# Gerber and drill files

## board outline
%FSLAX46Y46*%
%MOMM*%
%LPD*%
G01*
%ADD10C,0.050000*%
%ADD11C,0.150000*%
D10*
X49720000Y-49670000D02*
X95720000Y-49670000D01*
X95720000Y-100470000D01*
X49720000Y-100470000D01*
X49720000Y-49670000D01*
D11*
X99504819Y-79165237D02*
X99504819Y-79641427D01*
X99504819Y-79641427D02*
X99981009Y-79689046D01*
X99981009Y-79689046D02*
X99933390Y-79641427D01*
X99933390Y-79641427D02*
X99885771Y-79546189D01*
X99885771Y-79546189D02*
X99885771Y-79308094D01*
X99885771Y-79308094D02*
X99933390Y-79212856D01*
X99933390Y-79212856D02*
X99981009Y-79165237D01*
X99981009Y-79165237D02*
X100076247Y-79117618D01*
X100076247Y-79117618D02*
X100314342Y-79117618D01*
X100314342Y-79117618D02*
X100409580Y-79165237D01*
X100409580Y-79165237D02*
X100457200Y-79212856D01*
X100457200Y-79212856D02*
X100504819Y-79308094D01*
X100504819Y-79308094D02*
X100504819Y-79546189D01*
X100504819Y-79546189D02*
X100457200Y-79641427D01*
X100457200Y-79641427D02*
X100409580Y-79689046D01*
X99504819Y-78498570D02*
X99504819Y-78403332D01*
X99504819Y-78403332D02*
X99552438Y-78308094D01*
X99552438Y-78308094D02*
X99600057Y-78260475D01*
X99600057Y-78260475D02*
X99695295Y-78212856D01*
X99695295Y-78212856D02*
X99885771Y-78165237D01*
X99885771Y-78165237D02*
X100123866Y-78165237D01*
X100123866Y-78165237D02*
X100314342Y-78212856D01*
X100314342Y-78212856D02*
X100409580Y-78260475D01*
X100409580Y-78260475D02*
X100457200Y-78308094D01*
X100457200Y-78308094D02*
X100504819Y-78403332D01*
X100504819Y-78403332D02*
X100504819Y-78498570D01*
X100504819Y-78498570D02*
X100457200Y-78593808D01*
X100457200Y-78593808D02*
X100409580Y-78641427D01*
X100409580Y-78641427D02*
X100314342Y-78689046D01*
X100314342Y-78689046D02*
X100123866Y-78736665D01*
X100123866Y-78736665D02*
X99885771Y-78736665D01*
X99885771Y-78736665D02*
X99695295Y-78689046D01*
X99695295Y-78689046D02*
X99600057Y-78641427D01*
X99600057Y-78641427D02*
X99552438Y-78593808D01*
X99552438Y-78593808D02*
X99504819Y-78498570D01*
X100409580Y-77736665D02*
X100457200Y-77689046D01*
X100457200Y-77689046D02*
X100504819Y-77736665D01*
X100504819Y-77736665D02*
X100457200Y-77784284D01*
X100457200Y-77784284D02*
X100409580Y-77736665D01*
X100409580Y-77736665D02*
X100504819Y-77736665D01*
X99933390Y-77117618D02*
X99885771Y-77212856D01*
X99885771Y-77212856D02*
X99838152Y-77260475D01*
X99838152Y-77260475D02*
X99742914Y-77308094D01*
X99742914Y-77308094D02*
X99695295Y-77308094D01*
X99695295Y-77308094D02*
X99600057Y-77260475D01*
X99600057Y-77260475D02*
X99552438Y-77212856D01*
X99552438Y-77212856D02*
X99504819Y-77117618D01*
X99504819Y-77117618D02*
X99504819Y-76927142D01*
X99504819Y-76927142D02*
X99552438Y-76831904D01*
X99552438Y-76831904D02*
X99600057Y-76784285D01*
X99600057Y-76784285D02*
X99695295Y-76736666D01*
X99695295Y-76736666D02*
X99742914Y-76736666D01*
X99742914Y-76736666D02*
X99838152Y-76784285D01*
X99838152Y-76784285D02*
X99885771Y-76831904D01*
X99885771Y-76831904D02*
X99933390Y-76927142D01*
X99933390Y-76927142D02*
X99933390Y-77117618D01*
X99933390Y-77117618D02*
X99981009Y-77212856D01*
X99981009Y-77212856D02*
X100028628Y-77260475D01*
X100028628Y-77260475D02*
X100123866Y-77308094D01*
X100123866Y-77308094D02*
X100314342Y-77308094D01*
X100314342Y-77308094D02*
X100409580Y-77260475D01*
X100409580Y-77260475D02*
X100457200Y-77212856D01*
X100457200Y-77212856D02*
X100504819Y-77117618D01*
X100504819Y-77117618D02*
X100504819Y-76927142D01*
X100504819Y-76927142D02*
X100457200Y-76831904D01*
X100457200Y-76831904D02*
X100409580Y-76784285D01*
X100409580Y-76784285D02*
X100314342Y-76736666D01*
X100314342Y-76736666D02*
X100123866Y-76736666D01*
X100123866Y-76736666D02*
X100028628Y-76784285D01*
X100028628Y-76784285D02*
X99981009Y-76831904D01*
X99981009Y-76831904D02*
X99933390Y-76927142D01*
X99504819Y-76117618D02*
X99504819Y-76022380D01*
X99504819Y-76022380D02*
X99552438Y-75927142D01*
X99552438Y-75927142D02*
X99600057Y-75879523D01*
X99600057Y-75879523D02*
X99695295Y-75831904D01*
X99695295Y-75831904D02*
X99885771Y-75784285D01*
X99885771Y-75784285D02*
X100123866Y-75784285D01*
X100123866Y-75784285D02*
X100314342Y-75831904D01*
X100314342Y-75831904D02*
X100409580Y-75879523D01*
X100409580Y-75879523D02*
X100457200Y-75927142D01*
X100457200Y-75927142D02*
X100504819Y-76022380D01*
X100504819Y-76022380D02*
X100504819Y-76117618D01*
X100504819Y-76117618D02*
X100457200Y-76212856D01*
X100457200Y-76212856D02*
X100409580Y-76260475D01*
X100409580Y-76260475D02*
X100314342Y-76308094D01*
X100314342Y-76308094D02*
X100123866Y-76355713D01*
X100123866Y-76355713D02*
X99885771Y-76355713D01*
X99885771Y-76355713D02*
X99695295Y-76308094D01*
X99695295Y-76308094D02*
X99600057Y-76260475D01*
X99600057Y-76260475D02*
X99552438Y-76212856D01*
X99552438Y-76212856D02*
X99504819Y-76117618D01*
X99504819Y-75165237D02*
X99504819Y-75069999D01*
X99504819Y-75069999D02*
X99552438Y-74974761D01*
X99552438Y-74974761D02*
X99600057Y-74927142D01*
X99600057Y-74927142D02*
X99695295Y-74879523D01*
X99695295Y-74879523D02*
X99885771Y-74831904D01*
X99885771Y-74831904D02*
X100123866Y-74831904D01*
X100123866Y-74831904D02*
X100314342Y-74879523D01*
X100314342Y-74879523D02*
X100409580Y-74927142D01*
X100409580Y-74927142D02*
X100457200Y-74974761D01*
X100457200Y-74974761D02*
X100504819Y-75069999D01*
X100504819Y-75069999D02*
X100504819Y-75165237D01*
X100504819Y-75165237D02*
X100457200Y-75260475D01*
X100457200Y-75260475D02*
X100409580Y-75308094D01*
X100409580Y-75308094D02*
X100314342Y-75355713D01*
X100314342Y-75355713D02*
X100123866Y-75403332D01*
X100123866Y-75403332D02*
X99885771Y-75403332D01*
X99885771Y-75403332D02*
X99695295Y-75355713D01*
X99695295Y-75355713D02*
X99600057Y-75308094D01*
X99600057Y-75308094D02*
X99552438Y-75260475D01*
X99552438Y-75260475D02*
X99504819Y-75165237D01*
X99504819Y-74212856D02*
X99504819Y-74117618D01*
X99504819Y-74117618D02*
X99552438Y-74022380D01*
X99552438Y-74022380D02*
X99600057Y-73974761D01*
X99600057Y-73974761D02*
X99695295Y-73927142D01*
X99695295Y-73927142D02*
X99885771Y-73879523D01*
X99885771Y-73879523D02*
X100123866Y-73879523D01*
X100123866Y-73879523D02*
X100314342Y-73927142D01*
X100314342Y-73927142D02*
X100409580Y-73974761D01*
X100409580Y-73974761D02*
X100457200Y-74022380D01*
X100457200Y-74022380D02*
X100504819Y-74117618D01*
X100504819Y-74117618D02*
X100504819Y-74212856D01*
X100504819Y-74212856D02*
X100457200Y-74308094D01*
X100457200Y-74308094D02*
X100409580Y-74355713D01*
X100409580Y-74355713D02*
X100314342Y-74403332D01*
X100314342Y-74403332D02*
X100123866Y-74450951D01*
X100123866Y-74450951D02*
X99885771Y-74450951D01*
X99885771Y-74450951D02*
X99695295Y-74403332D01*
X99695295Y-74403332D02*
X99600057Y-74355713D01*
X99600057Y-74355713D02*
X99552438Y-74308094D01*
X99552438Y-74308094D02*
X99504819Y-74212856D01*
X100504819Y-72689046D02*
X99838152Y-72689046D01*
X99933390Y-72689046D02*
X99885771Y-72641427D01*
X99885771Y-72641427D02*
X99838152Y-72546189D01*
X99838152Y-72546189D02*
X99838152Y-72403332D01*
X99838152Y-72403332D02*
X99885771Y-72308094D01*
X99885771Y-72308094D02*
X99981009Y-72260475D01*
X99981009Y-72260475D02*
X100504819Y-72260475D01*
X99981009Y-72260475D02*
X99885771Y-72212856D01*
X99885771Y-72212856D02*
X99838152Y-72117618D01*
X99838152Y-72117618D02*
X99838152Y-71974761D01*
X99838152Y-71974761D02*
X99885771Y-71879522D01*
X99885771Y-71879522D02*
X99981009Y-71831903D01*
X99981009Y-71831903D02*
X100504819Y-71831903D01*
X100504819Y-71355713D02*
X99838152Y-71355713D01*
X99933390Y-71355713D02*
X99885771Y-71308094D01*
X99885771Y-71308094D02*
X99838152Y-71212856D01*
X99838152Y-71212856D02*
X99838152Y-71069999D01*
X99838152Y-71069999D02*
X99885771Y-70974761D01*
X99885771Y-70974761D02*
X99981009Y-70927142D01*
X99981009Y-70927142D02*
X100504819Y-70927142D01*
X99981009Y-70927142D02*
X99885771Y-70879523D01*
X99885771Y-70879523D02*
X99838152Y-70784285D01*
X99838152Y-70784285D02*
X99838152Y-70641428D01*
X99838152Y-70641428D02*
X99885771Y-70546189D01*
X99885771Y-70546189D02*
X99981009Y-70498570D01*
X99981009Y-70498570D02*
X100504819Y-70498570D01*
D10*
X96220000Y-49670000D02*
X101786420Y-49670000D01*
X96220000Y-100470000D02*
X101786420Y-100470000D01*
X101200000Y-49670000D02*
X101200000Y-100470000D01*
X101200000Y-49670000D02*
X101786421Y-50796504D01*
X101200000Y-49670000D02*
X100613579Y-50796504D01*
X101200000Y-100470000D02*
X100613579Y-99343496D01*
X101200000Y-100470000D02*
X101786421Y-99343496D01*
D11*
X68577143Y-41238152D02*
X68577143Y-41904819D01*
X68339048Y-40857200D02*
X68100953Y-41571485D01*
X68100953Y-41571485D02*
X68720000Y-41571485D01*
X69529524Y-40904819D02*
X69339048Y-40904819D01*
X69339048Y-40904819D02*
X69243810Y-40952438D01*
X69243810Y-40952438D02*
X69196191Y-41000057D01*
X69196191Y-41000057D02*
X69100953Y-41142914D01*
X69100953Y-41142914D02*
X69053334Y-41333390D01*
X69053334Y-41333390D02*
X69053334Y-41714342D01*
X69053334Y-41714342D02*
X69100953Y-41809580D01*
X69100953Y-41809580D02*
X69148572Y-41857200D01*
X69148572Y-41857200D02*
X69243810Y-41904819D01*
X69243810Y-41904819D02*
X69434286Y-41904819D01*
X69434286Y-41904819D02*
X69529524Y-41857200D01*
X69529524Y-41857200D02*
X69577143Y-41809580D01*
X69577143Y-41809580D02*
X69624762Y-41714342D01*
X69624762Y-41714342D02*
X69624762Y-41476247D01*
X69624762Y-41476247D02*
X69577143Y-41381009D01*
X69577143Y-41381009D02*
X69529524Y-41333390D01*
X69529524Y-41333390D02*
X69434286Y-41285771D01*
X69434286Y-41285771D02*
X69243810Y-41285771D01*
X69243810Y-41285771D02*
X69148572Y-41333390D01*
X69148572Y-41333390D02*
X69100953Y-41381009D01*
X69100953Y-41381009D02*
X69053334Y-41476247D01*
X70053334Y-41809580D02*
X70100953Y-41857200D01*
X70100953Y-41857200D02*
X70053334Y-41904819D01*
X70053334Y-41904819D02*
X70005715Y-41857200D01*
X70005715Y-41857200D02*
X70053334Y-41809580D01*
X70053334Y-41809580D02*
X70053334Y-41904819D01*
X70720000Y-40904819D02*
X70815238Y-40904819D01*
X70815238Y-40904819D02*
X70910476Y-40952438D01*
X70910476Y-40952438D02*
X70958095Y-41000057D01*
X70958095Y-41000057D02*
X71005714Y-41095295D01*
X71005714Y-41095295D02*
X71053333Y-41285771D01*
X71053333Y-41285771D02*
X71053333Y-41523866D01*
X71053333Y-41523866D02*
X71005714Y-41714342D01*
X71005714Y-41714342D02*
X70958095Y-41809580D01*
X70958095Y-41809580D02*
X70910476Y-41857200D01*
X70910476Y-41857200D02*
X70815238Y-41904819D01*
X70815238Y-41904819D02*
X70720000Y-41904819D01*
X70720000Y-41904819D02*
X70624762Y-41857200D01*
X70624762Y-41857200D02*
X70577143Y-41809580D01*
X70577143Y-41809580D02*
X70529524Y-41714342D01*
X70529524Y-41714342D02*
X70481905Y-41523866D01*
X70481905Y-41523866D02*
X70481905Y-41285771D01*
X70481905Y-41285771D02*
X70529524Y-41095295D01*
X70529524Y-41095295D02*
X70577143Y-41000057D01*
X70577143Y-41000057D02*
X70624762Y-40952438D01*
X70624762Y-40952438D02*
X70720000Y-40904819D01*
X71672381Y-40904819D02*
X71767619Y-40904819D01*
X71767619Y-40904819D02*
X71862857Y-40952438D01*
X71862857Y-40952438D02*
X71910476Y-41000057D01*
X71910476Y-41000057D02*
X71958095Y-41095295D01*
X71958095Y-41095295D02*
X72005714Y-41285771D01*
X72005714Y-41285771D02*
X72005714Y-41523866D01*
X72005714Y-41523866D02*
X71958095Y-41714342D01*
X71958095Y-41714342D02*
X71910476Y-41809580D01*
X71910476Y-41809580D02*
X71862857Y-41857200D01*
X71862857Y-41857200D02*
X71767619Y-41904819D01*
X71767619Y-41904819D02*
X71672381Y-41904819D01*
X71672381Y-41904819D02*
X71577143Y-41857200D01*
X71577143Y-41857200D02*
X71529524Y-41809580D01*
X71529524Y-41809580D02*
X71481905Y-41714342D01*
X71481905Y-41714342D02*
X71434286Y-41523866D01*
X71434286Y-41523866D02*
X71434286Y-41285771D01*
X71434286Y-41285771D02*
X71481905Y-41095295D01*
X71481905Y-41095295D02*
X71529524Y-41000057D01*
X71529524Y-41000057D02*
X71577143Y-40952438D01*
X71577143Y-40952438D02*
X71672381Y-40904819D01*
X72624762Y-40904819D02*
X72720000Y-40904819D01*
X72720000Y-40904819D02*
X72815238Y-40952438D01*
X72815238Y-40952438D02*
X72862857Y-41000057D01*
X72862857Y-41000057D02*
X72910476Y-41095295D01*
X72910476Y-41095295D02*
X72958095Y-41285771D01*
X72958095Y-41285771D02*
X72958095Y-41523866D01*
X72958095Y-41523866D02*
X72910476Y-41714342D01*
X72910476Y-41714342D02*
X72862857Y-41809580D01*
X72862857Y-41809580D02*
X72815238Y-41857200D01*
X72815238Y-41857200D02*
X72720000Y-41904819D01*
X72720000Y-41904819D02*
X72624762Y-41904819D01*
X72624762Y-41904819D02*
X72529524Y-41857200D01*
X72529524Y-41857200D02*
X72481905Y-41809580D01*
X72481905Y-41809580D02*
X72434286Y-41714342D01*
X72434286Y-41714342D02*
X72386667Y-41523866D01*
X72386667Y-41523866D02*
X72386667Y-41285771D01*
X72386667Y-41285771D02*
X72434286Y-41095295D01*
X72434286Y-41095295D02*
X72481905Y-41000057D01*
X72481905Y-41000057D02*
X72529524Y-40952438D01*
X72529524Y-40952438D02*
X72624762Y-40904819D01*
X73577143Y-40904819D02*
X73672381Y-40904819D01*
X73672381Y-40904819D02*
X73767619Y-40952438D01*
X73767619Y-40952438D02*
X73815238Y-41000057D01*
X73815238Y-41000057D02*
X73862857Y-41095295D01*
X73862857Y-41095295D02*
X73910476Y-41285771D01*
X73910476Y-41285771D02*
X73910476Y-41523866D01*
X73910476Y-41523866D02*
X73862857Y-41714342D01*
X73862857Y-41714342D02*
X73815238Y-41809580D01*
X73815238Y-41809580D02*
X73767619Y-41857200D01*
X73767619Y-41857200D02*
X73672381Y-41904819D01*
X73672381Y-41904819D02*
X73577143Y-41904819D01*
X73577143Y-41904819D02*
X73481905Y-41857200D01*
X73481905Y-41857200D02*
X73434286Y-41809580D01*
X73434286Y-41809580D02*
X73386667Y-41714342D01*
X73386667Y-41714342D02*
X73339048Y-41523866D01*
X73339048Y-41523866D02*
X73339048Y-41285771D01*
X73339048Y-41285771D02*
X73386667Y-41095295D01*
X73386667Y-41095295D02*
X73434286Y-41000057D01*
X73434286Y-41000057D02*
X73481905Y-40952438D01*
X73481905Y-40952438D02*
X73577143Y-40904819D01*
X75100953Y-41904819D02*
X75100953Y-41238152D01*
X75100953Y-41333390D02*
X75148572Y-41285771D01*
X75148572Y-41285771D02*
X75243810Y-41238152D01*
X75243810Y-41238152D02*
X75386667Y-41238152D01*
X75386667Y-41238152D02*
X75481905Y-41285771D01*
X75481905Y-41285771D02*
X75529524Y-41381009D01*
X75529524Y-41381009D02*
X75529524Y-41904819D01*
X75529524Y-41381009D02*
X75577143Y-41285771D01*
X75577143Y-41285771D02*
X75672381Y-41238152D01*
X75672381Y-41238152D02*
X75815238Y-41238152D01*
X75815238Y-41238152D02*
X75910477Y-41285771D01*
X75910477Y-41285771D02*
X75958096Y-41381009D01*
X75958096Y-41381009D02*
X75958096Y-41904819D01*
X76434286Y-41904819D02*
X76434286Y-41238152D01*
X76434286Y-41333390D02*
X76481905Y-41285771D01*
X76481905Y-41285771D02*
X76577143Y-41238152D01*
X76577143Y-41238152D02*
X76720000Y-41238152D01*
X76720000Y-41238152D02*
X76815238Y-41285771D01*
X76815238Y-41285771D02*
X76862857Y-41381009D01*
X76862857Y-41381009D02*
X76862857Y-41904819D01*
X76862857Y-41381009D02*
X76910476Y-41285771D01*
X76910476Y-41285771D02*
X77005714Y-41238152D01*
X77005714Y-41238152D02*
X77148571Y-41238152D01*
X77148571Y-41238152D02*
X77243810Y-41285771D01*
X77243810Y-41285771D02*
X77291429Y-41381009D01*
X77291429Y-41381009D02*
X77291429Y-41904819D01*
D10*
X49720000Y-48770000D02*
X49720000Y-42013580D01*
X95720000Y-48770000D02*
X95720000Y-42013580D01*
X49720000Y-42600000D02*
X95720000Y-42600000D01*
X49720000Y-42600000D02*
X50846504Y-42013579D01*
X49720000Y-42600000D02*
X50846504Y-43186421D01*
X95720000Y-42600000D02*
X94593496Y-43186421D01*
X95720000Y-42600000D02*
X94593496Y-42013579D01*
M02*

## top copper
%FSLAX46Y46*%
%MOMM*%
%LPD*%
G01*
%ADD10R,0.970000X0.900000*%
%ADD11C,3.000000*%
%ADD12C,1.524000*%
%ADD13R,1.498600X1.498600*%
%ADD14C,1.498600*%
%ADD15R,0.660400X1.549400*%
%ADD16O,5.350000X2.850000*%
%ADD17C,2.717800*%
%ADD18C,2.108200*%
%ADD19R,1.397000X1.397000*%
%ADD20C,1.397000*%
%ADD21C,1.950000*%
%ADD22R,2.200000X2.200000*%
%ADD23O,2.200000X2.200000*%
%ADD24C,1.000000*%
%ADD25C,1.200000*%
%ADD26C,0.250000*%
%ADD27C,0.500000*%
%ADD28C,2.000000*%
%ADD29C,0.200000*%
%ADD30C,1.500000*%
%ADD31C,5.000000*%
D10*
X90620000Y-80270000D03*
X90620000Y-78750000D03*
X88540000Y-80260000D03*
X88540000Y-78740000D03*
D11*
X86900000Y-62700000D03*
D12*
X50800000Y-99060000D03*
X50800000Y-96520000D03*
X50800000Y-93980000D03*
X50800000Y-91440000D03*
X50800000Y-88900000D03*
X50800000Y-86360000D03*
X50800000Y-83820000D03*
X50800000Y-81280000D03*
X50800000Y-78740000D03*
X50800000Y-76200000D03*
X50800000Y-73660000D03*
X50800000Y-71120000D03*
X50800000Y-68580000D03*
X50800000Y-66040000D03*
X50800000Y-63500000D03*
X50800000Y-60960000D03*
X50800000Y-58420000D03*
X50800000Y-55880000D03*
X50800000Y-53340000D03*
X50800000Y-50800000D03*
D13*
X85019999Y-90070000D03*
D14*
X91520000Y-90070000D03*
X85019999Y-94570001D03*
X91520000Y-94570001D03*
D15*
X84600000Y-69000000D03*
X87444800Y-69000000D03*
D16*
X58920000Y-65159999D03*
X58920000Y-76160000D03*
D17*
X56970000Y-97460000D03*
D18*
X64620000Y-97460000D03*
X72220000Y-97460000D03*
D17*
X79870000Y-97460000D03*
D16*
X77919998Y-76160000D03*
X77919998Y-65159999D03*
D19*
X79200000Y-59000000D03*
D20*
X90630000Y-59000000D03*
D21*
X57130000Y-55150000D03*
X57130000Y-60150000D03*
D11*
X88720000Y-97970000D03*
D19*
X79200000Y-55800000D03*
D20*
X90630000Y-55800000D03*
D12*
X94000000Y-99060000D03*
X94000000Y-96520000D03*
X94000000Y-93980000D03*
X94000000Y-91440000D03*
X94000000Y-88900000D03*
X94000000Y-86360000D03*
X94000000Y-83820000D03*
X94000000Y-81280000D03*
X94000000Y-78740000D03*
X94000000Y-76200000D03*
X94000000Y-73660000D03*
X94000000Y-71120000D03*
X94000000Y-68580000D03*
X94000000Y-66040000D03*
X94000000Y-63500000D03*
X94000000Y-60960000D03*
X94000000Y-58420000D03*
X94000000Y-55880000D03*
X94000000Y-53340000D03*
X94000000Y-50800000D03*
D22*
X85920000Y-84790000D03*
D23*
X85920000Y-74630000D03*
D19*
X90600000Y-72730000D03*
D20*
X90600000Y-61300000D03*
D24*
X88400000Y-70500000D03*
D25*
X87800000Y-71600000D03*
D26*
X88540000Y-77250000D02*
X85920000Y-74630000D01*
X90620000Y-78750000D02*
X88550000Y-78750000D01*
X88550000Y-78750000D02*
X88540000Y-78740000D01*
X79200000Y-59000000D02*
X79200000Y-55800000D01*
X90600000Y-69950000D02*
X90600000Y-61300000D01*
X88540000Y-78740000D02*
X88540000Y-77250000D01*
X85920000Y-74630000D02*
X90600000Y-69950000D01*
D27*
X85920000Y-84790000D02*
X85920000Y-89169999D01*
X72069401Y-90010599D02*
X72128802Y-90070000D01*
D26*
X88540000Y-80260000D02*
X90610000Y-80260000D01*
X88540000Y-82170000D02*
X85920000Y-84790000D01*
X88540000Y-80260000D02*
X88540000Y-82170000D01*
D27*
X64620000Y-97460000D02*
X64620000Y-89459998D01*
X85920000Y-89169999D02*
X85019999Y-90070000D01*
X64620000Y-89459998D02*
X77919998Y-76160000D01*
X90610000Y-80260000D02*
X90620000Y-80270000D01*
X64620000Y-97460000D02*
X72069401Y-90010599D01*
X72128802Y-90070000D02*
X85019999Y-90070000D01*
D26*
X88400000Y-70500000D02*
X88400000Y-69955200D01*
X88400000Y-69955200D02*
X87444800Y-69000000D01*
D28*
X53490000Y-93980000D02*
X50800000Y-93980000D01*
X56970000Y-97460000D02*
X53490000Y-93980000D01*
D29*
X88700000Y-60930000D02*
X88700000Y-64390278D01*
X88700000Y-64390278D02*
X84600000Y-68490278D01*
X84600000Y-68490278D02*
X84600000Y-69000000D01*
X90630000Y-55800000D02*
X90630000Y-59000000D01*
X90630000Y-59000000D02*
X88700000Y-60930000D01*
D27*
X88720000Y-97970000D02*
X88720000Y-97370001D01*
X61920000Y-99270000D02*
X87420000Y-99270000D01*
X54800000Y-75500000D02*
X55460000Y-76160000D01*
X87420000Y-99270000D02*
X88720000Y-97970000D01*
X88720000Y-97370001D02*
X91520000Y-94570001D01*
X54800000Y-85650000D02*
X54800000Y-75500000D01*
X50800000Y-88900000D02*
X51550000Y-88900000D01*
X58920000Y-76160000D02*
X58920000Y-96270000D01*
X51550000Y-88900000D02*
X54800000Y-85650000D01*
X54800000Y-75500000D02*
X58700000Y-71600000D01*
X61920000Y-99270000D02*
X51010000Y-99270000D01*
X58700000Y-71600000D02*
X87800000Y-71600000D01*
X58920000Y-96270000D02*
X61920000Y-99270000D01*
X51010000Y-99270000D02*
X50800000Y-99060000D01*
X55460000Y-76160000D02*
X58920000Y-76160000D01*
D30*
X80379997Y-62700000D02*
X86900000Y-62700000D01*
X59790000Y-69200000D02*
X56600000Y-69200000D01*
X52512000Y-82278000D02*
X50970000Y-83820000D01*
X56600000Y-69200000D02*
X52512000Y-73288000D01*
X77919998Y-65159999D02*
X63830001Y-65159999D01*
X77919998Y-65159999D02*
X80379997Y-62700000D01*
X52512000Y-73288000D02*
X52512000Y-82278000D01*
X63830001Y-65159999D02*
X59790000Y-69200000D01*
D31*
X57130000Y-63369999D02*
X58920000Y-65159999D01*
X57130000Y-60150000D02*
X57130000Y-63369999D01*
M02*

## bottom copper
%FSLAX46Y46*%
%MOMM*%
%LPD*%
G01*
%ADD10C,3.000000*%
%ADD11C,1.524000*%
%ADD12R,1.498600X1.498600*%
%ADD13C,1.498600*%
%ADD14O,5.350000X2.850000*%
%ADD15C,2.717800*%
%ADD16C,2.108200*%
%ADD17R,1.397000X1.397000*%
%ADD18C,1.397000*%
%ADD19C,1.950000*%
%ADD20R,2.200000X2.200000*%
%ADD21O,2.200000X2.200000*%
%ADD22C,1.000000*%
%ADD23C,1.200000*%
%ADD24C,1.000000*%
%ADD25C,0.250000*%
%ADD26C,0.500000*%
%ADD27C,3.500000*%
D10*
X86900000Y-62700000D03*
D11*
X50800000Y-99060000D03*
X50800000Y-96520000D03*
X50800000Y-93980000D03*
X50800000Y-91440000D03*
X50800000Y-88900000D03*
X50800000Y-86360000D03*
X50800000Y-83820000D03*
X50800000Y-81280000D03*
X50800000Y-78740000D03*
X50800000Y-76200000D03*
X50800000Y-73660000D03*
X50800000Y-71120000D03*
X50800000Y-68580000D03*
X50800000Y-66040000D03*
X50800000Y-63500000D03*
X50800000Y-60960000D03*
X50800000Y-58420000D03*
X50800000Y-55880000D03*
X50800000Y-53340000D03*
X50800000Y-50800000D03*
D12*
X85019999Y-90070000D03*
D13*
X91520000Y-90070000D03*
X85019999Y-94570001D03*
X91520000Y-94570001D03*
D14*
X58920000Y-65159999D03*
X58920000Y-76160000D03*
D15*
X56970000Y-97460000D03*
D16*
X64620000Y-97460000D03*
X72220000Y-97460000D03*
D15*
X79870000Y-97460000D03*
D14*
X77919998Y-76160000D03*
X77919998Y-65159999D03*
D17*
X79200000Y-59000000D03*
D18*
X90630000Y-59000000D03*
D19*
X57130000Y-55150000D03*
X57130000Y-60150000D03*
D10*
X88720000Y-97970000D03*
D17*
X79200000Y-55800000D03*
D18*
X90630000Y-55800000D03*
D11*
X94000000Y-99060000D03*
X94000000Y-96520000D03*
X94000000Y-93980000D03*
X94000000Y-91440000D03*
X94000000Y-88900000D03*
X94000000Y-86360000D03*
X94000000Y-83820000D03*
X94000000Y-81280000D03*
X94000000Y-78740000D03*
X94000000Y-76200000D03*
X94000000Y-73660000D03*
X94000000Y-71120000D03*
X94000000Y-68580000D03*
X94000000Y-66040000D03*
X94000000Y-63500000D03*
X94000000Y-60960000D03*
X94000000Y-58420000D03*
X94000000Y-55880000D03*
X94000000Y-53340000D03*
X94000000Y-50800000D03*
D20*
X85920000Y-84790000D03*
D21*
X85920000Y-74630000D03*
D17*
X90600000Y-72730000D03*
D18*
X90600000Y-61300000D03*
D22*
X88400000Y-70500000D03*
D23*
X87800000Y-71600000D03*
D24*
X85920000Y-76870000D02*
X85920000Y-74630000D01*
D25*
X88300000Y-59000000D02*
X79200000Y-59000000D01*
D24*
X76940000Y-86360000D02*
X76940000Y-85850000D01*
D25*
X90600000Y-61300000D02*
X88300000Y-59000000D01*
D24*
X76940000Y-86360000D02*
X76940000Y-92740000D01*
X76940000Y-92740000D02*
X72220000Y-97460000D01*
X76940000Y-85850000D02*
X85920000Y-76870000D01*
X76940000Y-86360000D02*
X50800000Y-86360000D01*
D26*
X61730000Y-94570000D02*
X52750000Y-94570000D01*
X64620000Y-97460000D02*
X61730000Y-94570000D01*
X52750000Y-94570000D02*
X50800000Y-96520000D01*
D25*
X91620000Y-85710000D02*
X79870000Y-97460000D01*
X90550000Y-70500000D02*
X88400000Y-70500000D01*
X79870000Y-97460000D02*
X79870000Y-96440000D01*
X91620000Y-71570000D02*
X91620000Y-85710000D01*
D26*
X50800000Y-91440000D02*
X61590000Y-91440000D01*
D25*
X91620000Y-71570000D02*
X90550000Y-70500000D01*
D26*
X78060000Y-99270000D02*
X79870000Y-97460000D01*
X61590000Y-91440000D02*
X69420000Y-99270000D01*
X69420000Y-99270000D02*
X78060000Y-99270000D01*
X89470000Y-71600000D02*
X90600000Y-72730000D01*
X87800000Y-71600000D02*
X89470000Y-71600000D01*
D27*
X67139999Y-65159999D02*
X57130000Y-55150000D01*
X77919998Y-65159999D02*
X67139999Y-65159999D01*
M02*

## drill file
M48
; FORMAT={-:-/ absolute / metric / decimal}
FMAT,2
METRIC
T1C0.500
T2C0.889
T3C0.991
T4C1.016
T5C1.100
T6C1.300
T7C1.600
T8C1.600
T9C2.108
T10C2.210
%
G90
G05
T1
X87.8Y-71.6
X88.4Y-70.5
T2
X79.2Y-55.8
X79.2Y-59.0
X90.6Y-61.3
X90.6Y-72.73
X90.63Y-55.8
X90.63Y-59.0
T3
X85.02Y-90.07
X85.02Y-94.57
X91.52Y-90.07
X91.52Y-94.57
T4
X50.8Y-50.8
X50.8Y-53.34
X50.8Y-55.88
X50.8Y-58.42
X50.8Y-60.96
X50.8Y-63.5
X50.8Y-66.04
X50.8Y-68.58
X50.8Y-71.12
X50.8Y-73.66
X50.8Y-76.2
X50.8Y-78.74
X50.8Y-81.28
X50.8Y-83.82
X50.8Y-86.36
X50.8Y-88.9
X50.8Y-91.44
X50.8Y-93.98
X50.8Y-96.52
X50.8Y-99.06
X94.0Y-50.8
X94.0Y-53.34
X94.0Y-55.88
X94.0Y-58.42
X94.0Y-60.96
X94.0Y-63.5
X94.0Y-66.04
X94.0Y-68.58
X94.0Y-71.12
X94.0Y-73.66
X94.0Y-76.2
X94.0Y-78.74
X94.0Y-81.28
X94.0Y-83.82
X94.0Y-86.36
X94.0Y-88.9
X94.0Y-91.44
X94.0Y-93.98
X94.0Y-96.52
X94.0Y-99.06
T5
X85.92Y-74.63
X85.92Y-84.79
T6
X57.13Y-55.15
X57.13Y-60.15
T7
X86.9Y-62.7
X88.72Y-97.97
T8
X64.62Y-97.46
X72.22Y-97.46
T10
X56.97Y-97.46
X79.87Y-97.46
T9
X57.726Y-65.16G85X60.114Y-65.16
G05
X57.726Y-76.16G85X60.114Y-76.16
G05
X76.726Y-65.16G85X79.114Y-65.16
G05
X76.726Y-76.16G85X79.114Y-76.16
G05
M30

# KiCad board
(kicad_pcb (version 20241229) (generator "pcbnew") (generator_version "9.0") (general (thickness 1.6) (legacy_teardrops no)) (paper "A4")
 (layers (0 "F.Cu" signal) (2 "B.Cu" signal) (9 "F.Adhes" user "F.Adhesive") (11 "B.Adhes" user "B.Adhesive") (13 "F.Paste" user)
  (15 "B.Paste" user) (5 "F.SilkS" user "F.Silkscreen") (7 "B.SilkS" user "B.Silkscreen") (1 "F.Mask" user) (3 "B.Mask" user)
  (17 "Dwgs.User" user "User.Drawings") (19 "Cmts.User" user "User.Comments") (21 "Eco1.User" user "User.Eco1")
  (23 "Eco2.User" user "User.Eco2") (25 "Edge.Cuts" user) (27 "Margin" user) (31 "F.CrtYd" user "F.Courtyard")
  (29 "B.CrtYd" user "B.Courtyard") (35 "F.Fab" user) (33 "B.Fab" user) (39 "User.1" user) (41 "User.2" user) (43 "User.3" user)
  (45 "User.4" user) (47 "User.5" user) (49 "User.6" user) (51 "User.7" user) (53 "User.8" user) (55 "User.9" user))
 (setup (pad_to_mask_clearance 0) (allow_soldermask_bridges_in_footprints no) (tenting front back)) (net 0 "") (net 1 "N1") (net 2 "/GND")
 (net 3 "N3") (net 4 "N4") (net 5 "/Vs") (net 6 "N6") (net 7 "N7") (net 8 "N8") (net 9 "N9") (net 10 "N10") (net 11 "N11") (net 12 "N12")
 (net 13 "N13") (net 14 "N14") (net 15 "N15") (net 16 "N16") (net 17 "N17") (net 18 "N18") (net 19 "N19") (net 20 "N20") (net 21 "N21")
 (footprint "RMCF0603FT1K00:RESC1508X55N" (layer "F.Cu") (at 90.62 79.51 90)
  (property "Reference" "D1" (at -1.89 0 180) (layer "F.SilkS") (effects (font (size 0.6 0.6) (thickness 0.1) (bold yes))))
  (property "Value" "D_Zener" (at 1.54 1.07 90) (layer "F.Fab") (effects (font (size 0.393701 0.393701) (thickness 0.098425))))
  (pad "1" smd rect (at -0.76 0 90) (size 0.9 0.97) (layers "F.Cu" "F.Mask" "F.Paste") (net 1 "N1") (solder_mask_margin 0.102))
  (pad "2" smd rect (at 0.76 0 90) (size 0.9 0.97) (layers "F.Cu" "F.Mask" "F.Paste") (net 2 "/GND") (solder_mask_margin 0.102)))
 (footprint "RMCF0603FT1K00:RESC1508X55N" (layer "F.Cu") (at 88.54 79.5 90)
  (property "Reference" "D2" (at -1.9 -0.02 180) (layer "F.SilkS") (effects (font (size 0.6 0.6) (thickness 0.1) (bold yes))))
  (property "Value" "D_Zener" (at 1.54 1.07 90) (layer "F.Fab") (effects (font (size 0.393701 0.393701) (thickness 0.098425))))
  (pad "1" smd rect (at -0.76 0 90) (size 0.9 0.97) (layers "F.Cu" "F.Mask" "F.Paste") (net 1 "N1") (solder_mask_margin 0.102))
  (pad "2" smd rect (at 0.76 0 90) (size 0.9 0.97) (layers "F.Cu" "F.Mask" "F.Paste") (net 2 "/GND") (solder_mask_margin 0.102)))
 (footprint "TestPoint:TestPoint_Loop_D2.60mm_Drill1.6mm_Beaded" (layer "F.Cu") (at 86.9 62.7)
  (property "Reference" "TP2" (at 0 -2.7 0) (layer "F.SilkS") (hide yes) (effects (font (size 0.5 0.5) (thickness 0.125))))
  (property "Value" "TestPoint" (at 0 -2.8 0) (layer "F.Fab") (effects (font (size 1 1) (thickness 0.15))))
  (pad "1" thru_hole circle (at 0 0) (size 3 3) (drill 1.6) (layers "*.Cu" "*.Mask") (remove_unused_layers no) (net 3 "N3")))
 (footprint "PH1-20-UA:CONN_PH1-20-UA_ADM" (layer "F.Cu") (at 50.8 99.06 90)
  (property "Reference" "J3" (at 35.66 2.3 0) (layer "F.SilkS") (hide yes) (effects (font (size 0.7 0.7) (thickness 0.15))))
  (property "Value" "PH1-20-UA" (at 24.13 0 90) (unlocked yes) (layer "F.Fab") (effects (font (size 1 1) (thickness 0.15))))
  (pad "1" thru_hole circle (at 0 0 90) (size 1.524 1.524) (drill 1.016) (layers "*.Cu" "*.Mask") (remove_unused_layers no) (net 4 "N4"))
  (pad "2" thru_hole circle (at 2.54 0 90) (size 1.524 1.524) (drill 1.016) (layers "*.Cu" "*.Mask") (remove_unused_layers no) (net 1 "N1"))
  (pad "3" thru_hole circle (at 5.08 0 90) (size 1.524 1.524) (drill 1.016) (layers "*.Cu" "*.Mask") (remove_unused_layers no) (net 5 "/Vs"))
  (pad "4" thru_hole circle (at 7.62 0 90) (size 1.524 1.524) (drill 1.016) (layers "*.Cu" "*.Mask") (remove_unused_layers no) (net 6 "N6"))
  (pad "5" thru_hole circle (at 10.16 0 90) (size 1.524 1.524) (drill 1.016) (layers "*.Cu" "*.Mask") (remove_unused_layers no) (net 4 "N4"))
  (pad "6" thru_hole circle (at 12.7 0 90) (size 1.524 1.524) (drill 1.016) (layers "*.Cu" "*.Mask") (remove_unused_layers no)
   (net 2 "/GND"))
  (pad "7" thru_hole circle (at 15.24 0 90) (size 1.524 1.524) (drill 1.016) (layers "*.Cu" "*.Mask") (remove_unused_layers no) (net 3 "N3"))
  (pad "8" thru_hole circle (at 17.78 0 90) (size 1.524 1.524) (drill 1.016) (layers "*.Cu" "*.Mask") (remove_unused_layers no) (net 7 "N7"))
  (pad "9" thru_hole circle (at 20.32 0 90) (size 1.524 1.524) (drill 1.016) (layers "*.Cu" "*.Mask") (remove_unused_layers no) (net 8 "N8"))
  (pad "10" thru_hole circle (at 22.86 0 90) (size 1.524 1.524) (drill 1.016) (layers "*.Cu" "*.Mask") (remove_unused_layers no)
   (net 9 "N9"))
  (pad "11" thru_hole circle (at 25.4 0 90) (size 1.524 1.524) (drill 1.016) (layers "*.Cu" "*.Mask") (remove_unused_layers no)
   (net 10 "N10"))
  (pad "12" thru_hole circle (at 27.94 0 90) (size 1.524 1.524) (drill 1.016) (layers "*.Cu" "*.Mask") (remove_unused_layers no)
   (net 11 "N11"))
  (pad "13" thru_hole circle (at 30.48 0 90) (size 1.524 1.524) (drill 1.016) (layers "*.Cu" "*.Mask") (remove_unused_layers no)
   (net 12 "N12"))
  (pad "14" thru_hole circle (at 33.02 0 90) (size 1.524 1.524) (drill 1.016) (layers "*.Cu" "*.Mask") (remove_unused_layers no)
   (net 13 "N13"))
  (pad "15" thru_hole circle (at 35.56 0 90) (size 1.524 1.524) (drill 1.016) (layers "*.Cu" "*.Mask") (remove_unused_layers no)
   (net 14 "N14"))
  (pad "16" thru_hole circle (at 38.1 0 90) (size 1.524 1.524) (drill 1.016) (layers "*.Cu" "*.Mask") (remove_unused_layers no)
   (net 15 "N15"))
  (pad "17" thru_hole circle (at 40.64 0 90) (size 1.524 1.524) (drill 1.016) (layers "*.Cu" "*.Mask") (remove_unused_layers no)
   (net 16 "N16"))
  (pad "18" thru_hole circle (at 43.18 0 90) (size 1.524 1.524) (drill 1.016) (layers "*.Cu" "*.Mask") (remove_unused_layers no)
   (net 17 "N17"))
  (pad "19" thru_hole circle (at 45.72 0 90) (size 1.524 1.524) (drill 1.016) (layers "*.Cu" "*.Mask") (remove_unused_layers no)
   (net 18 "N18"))
  (pad "20" thru_hole circle (at 48.26 0 90) (size 1.524 1.524) (drill 1.016) (layers "*.Cu" "*.Mask") (remove_unused_layers no)
   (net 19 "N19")))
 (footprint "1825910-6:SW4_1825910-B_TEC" (layer "F.Cu") (at 91.52 94.570001)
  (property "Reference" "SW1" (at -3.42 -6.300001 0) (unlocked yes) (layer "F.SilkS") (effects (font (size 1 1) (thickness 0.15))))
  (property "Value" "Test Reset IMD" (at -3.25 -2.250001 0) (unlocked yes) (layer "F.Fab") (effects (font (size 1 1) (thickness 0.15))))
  (pad "1" thru_hole rect (at -6.500001 -4.500001) (size 1.4986 1.4986) (drill 0.9906) (layers "*.Cu" "*.Mask") (remove_unused_layers no)
   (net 1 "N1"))
  (pad "2" thru_hole circle (at 0 -4.500001) (size 1.4986 1.4986) (drill 0.9906) (layers "*.Cu" "*.Mask") (remove_unused_layers no)
   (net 4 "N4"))
  (pad "3" thru_hole circle (at -6.500001 0) (size 1.4986 1.4986) (drill 0.9906) (layers "*.Cu" "*.Mask") (remove_unused_layers no))
  (pad "4" thru_hole circle (at 0 0) (size 1.4986 1.4986) (drill 0.9906) (layers "*.Cu" "*.Mask") (remove_unused_layers no)))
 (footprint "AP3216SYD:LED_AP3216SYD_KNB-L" (layer "F.Cu") (at 86.0224 69)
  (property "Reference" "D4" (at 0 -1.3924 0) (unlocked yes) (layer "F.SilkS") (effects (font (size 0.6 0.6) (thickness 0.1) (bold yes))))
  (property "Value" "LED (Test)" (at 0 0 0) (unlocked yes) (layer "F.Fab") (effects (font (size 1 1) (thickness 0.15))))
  (pad "1" smd rect (at -1.4224 0) (size 0.6604 1.5494) (layers "F.Cu" "F.Mask" "F.Paste") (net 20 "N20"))
  (pad "2" smd rect (at 1.4224 0) (size 0.6604 1.5494) (layers "F.Cu" "F.Mask" "F.Paste") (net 6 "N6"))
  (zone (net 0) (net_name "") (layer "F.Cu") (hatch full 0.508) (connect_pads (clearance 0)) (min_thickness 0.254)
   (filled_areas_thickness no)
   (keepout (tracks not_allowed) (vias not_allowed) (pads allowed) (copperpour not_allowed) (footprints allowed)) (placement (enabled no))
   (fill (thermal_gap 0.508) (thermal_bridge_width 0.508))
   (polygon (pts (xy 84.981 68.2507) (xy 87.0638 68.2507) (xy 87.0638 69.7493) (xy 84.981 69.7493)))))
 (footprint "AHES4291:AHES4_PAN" (layer "F.Cu") (at 58.919999 65.159998)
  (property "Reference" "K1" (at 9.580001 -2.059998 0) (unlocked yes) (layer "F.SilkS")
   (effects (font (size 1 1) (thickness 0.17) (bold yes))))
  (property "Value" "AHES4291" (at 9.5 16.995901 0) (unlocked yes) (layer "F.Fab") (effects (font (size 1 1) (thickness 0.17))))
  (pad "1" thru_hole oval (at 0.000001 0.000001) (size 5.35 2.85) (drill oval 4.4958 2.1082) (layers "*.Cu" "*.Mask")
   (remove_unused_layers no) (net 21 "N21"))
  (pad "2" thru_hole oval (at 0.000001 11.000002) (size 5.35 2.85) (drill oval 4.4958 2.1082) (layers "*.Cu" "*.Mask")
   (remove_unused_layers no) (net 4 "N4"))
  (pad "3" thru_hole circle (at -1.949999 32.300002) (size 2.7178 2.7178) (drill 2.2098) (layers "*.Cu" "*.Mask") (remove_unused_layers no)
   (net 5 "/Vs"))
  (pad "4" thru_hole circle (at 5.700001 32.300002) (size 2.1082 2.1082) (drill 1.6002) (layers "*.Cu" "*.Mask") (remove_unused_layers no)
   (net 1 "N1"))
  (pad "5" thru_hole circle (at 13.300001 32.300002) (size 2.1082 2.1082) (drill 1.6002) (layers "*.Cu" "*.Mask") (remove_unused_layers no)
   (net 2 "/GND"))
  (pad "6" thru_hole circle (at 20.950001 32.300002) (size 2.7178 2.7178) (drill 2.2098) (layers "*.Cu" "*.Mask") (remove_unused_layers no)
   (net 6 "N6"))
  (pad "7" thru_hole oval (at 18.999999 11.000002) (size 5.35 2.85) (drill oval 4.4958 2.1082) (layers "*.Cu" "*.Mask")
   (remove_unused_layers no) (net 1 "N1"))
  (pad "8" thru_hole oval (at 18.999999 0.000001) (size 5.35 2.85) (drill oval 4.4958 2.1082) (layers "*.Cu" "*.Mask")
   (remove_unused_layers no) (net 3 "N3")))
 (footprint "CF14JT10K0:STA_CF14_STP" (layer "F.Cu") (at 79.2 59)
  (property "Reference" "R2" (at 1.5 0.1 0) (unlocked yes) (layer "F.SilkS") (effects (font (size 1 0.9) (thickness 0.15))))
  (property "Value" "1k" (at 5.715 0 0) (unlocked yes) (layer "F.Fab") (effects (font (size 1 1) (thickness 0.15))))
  (pad "1" thru_hole rect (at 0 0) (size 1.397 1.397) (drill 0.889) (layers "*.Cu" "*.Mask") (remove_unused_layers no) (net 2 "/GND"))
  (pad "2" thru_hole circle (at 11.43 0) (size 1.397 1.397) (drill 0.889) (layers "*.Cu" "*.Mask") (remove_unused_layers no) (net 20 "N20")))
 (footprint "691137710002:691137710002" (layer "F.Cu") (at 57.13 57.65 -90)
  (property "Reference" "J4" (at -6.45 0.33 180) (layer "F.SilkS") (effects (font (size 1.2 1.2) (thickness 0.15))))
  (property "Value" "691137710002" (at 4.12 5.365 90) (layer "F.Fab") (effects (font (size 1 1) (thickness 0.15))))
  (pad "1" thru_hole circle (at -2.5 0 270) (size 1.95 1.95) (drill 1.3) (layers "*.Cu" "*.Mask") (remove_unused_layers no) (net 3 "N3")
   (solder_mask_margin 0.102))
  (pad "2" thru_hole circle (at 2.5 0 270) (size 1.95 1.95) (drill 1.3) (layers "*.Cu" "*.Mask") (remove_unused_layers no) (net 21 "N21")
   (solder_mask_margin 0.102)))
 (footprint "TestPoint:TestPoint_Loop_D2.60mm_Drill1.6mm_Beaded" (layer "F.Cu") (at 88.72 97.97)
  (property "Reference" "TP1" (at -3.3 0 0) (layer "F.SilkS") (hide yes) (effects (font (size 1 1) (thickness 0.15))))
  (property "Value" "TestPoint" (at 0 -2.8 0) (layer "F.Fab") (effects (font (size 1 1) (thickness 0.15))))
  (pad "1" thru_hole circle (at 0 0) (size 3 3) (drill 1.6) (layers "*.Cu" "*.Mask") (remove_unused_layers no) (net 4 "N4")))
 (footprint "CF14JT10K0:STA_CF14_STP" (layer "F.Cu") (at 79.2 55.8)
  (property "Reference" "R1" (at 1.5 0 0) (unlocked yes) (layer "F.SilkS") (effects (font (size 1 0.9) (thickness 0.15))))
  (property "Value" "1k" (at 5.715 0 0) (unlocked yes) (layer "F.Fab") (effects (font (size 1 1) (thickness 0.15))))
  (pad "1" thru_hole rect (at 0 0) (size 1.397 1.397) (drill 0.889) (layers "*.Cu" "*.Mask") (remove_unused_layers no) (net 2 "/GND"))
  (pad "2" thru_hole circle (at 11.43 0) (size 1.397 1.397) (drill 0.889) (layers "*.Cu" "*.Mask") (remove_unused_layers no) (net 20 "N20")))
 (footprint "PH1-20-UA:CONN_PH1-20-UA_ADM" (layer "F.Cu") (at 94 99.06 90)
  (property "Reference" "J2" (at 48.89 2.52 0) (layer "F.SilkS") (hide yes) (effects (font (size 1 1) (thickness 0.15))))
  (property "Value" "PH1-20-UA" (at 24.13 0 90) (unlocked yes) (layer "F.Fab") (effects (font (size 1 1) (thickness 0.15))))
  (pad "1" thru_hole circle (at 0 0 90) (size 1.524 1.524) (drill 1.016) (layers "*.Cu" "*.Mask") (remove_unused_layers no))
  (pad "2" thru_hole circle (at 2.54 0 90) (size 1.524 1.524) (drill 1.016) (layers "*.Cu" "*.Mask") (remove_unused_layers no))
  (pad "3" thru_hole circle (at 5.08 0 90) (size 1.524 1.524) (drill 1.016) (layers "*.Cu" "*.Mask") (remove_unused_layers no))
  (pad "4" thru_hole circle (at 7.62 0 90) (size 1.524 1.524) (drill 1.016) (layers "*.Cu" "*.Mask") (remove_unused_layers no))
  (pad "5" thru_hole circle (at 10.16 0 90) (size 1.524 1.524) (drill 1.016) (layers "*.Cu" "*.Mask") (remove_unused_layers no))
  (pad "6" thru_hole circle (at 12.7 0 90) (size 1.524 1.524) (drill 1.016) (layers "*.Cu" "*.Mask") (remove_unused_layers no))
  (pad "7" thru_hole circle (at 15.24 0 90) (size 1.524 1.524) (drill 1.016) (layers "*.Cu" "*.Mask") (remove_unused_layers no))
  (pad "8" thru_hole circle (at 17.78 0 90) (size 1.524 1.524) (drill 1.016) (layers "*.Cu" "*.Mask") (remove_unused_layers no))
  (pad "9" thru_hole circle (at 20.32 0 90) (size 1.524 1.524) (drill 1.016) (layers "*.Cu" "*.Mask") (remove_unused_layers no))
  (pad "10" thru_hole circle (at 22.86 0 90) (size 1.524 1.524) (drill 1.016) (layers "*.Cu" "*.Mask") (remove_unused_layers no))
  (pad "11" thru_hole circle (at 25.4 0 90) (size 1.524 1.524) (drill 1.016) (layers "*.Cu" "*.Mask") (remove_unused_layers no))
  (pad "12" thru_hole circle (at 27.94 0 90) (size 1.524 1.524) (drill 1.016) (layers "*.Cu" "*.Mask") (remove_unused_layers no))
  (pad "13" thru_hole circle (at 30.48 0 90) (size 1.524 1.524) (drill 1.016) (layers "*.Cu" "*.Mask") (remove_unused_layers no))
  (pad "14" thru_hole circle (at 33.02 0 90) (size 1.524 1.524) (drill 1.016) (layers "*.Cu" "*.Mask") (remove_unused_layers no))
  (pad "15" thru_hole circle (at 35.56 0 90) (size 1.524 1.524) (drill 1.016) (layers "*.Cu" "*.Mask") (remove_unused_layers no))
  (pad "16" thru_hole circle (at 38.1 0 90) (size 1.524 1.524) (drill 1.016) (layers "*.Cu" "*.Mask") (remove_unused_layers no))
  (pad "17" thru_hole circle (at 40.64 0 90) (size 1.524 1.524) (drill 1.016) (layers "*.Cu" "*.Mask") (remove_unused_layers no))
  (pad "18" thru_hole circle (at 43.18 0 90) (size 1.524 1.524) (drill 1.016) (layers "*.Cu" "*.Mask") (remove_unused_layers no))
  (pad "19" thru_hole circle (at 45.72 0 90) (size 1.524 1.524) (drill 1.016) (layers "*.Cu" "*.Mask") (remove_unused_layers no))
  (pad "20" thru_hole circle (at 48.26 0 90) (size 1.524 1.524) (drill 1.016) (layers "*.Cu" "*.Mask") (remove_unused_layers no)))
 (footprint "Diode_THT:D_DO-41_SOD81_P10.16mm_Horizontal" (layer "F.Cu") (at 85.92 84.79 90)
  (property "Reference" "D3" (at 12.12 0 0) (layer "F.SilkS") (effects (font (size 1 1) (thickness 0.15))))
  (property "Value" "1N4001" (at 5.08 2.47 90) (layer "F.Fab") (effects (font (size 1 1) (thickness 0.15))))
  (pad "1" thru_hole rect (at 0 0 90) (size 2.2 2.2) (drill 1.1) (layers "*.Cu" "*.Mask") (remove_unused_layers no) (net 1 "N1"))
  (pad "2" thru_hole oval (at 10.16 0 90) (size 2.2 2.2) (drill 1.1) (layers "*.Cu" "*.Mask") (remove_unused_layers no) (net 2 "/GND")))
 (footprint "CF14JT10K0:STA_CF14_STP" (layer "F.Cu") (at 90.6 72.73 90)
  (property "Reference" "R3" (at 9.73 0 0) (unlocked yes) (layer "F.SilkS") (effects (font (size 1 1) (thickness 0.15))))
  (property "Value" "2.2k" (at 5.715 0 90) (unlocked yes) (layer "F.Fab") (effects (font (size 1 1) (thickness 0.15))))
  (pad "1" thru_hole rect (at 0 0 90) (size 1.397 1.397) (drill 0.889) (layers "*.Cu" "*.Mask") (remove_unused_layers no) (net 4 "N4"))
  (pad "2" thru_hole circle (at 11.43 0 90) (size 1.397 1.397) (drill 0.889) (layers "*.Cu" "*.Mask") (remove_unused_layers no)
   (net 2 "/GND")))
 (gr_rect (start 49.72 49.67) (end 95.72 100.47) (stroke (width 0.05) (type default)) (fill no) (layer "Edge.Cuts"))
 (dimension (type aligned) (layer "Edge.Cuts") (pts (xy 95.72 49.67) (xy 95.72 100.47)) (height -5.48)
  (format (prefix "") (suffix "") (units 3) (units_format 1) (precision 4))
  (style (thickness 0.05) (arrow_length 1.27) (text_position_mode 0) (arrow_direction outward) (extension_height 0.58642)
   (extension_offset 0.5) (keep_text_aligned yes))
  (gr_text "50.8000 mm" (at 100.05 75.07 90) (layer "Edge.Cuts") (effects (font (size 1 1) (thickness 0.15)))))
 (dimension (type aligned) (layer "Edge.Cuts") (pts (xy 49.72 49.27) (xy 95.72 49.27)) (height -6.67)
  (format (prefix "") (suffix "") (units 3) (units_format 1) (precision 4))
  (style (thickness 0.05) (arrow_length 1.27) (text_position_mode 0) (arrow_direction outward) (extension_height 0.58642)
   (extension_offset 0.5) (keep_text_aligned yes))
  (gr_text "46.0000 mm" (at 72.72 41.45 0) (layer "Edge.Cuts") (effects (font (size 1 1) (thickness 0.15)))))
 (segment (start 88.54 77.25) (end 85.92 74.63) (width 0.25) (layer "F.Cu") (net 2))
 (segment (start 90.62 78.75) (end 88.55 78.75) (width 0.25) (layer "F.Cu") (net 2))
 (segment (start 88.55 78.75) (end 88.54 78.74) (width 0.25) (layer "F.Cu") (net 2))
 (segment (start 79.2 59) (end 79.2 55.8) (width 0.25) (layer "F.Cu") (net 2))
 (segment (start 90.6 69.95) (end 90.6 61.3) (width 0.25) (layer "F.Cu") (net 2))
 (segment (start 88.54 78.74) (end 88.54 77.25) (width 0.25) (layer "F.Cu") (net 2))
 (segment (start 85.92 74.63) (end 90.6 69.95) (width 0.25) (layer "F.Cu") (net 2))
 (segment (start 85.92 76.87) (end 85.92 74.63) (width 1) (layer "B.Cu") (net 2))
 (segment (start 88.3 59) (end 79.2 59) (width 0.25) (layer "B.Cu") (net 2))
 (segment (start 76.94 86.36) (end 76.94 85.85) (width 1) (layer "B.Cu") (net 2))
 (segment (start 90.6 61.3) (end 88.3 59) (width 0.25) (layer "B.Cu") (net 2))
 (segment (start 76.94 86.36) (end 76.94 92.74) (width 1) (layer "B.Cu") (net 2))
 (segment (start 76.94 92.74) (end 72.22 97.46) (width 1) (layer "B.Cu") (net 2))
 (segment (start 76.94 85.85) (end 85.92 76.87) (width 1) (layer "B.Cu") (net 2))
 (segment (start 76.94 86.36) (end 50.8 86.36) (width 1) (layer "B.Cu") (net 2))
 (segment (start 85.92 84.79) (end 85.92 89.169999) (width 0.5) (layer "F.Cu") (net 1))
 (segment (start 72.069401 90.010599) (end 72.128802 90.07) (width 0.5) (layer "F.Cu") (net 1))
 (segment (start 88.54 80.26) (end 90.61 80.26) (width 0.25) (layer "F.Cu") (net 1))
 (segment (start 88.54 82.17) (end 85.92 84.79) (width 0.25) (layer "F.Cu") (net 1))
 (segment (start 88.54 80.26) (end 88.54 82.17) (width 0.25) (layer "F.Cu") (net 1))
 (segment (start 64.62 97.46) (end 64.62 89.459998) (width 0.5) (layer "F.Cu") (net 1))
 (segment (start 85.92 89.169999) (end 85.019999 90.07) (width 0.5) (layer "F.Cu") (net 1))
 (segment (start 64.62 89.459998) (end 77.919998 76.16) (width 0.5) (layer "F.Cu") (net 1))
 (segment (start 90.61 80.26) (end 90.62 80.27) (width 0.5) (layer "F.Cu") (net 1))
 (segment (start 64.62 97.46) (end 72.069401 90.010599) (width 0.5) (layer "F.Cu") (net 1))
 (segment (start 72.128802 90.07) (end 85.019999 90.07) (width 0.5) (layer "F.Cu") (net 1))
 (segment (start 61.73 94.57) (end 52.75 94.57) (width 0.5) (layer "B.Cu") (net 1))
 (segment (start 64.62 97.46) (end 61.73 94.57) (width 0.5) (layer "B.Cu") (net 1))
 (segment (start 52.75 94.57) (end 50.8 96.52) (width 0.5) (layer "B.Cu") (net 1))
 (segment (start 88.4 70.5) (end 88.4 69.9552) (width 0.25) (layer "F.Cu") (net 6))
 (segment (start 88.4 69.9552) (end 87.4448 69) (width 0.25) (layer "F.Cu") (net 6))
 (via (at 88.4 70.5) (size 1) (drill 0.5) (layers "F.Cu" "B.Cu") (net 6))
 (segment (start 91.62 85.71) (end 79.87 97.46) (width 0.25) (layer "B.Cu") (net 6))
 (segment (start 90.55 70.5) (end 88.4 70.5) (width 0.25) (layer "B.Cu") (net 6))
 (segment (start 79.87 97.46) (end 79.87 96.44) (width 0.25) (layer "B.Cu") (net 6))
 (segment (start 91.62 71.57) (end 91.62 85.71) (width 0.25) (layer "B.Cu") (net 6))
 (segment (start 50.8 91.44) (end 61.59 91.44) (width 0.5) (layer "B.Cu") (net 6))
 (segment (start 91.62 71.57) (end 90.55 70.5) (width 0.25) (layer "B.Cu") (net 6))
 (segment (start 78.06 99.27) (end 79.87 97.46) (width 0.5) (layer "B.Cu") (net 6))
 (segment (start 61.59 91.44) (end 69.42 99.27) (width 0.5) (layer "B.Cu") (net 6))
 (segment (start 69.42 99.27) (end 78.06 99.27) (width 0.5) (layer "B.Cu") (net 6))
 (segment (start 53.49 93.98) (end 50.8 93.98) (width 2) (layer "F.Cu") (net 5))
 (segment (start 56.97 97.46) (end 53.49 93.98) (width 2) (layer "F.Cu") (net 5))
 (segment (start 88.7 60.93) (end 88.7 64.390278) (width 0.2) (layer "F.Cu") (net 20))
 (segment (start 88.7 64.390278) (end 84.6 68.490278) (width 0.2) (layer "F.Cu") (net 20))
 (segment (start 84.6 68.490278) (end 84.6 69) (width 0.2) (layer "F.Cu") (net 20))
 (segment (start 90.63 55.8) (end 90.63 59) (width 0.2) (layer "F.Cu") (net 20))
 (segment (start 90.63 59) (end 88.7 60.93) (width 0.2) (layer "F.Cu") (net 20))
 (segment (start 88.72 97.97) (end 88.72 97.370001) (width 0.5) (layer "F.Cu") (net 4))
 (segment (start 61.92 99.27) (end 87.42 99.27) (width 0.5) (layer "F.Cu") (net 4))
 (segment (start 54.8 75.5) (end 55.46 76.16) (width 0.5) (layer "F.Cu") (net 4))
 (segment (start 87.42 99.27) (end 88.72 97.97) (width 0.5) (layer "F.Cu") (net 4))
 (segment (start 88.72 97.370001) (end 91.52 94.570001) (width 0.5) (layer "F.Cu") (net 4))
 (segment (start 54.8 85.65) (end 54.8 75.5) (width 0.5) (layer "F.Cu") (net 4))
 (segment (start 50.8 88.9) (end 51.55 88.9) (width 0.5) (layer "F.Cu") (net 4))
 (segment (start 58.92 76.16) (end 58.92 96.27) (width 0.5) (layer "F.Cu") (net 4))
 (segment (start 51.55 88.9) (end 54.8 85.65) (width 0.5) (layer "F.Cu") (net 4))
 (segment (start 54.8 75.5) (end 58.7 71.6) (width 0.5) (layer "F.Cu") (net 4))
 (segment (start 61.92 99.27) (end 51.01 99.27) (width 0.5) (layer "F.Cu") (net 4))
 (segment (start 58.7 71.6) (end 87.8 71.6) (width 0.5) (layer "F.Cu") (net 4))
 (segment (start 58.92 96.27) (end 61.92 99.27) (width 0.5) (layer "F.Cu") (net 4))
 (segment (start 51.01 99.27) (end 50.8 99.06) (width 0.5) (layer "F.Cu") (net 4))
 (segment (start 55.46 76.16) (end 58.92 76.16) (width 0.5) (layer "F.Cu") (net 4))
 (via (at 87.8 71.6) (size 1.2) (drill 0.5) (layers "F.Cu" "B.Cu") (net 4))
 (segment (start 89.47 71.6) (end 90.6 72.73) (width 0.5) (layer "B.Cu") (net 4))
 (segment (start 87.8 71.6) (end 89.47 71.6) (width 0.5) (layer "B.Cu") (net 4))
 (segment (start 80.379997 62.7) (end 86.9 62.7) (width 1.5) (layer "F.Cu") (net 3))
 (segment (start 59.79 69.2) (end 56.6 69.2) (width 1.5) (layer "F.Cu") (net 3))
 (segment (start 52.512 82.278) (end 50.97 83.82) (width 1.5) (layer "F.Cu") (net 3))
 (segment (start 56.6 69.2) (end 52.512 73.288) (width 1.5) (layer "F.Cu") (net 3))
 (segment (start 77.919998 65.159999) (end 63.830001 65.159999) (width 1.5) (layer "F.Cu") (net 3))
 (segment (start 77.919998 65.159999) (end 80.379997 62.7) (width 1.5) (layer "F.Cu") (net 3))
 (segment (start 52.512 73.288) (end 52.512 82.278) (width 1.5) (layer "F.Cu") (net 3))
 (segment (start 63.830001 65.159999) (end 59.79 69.2) (width 1.5) (layer "F.Cu") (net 3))
 (segment (start 67.139999 65.159999) (end 57.13 55.15) (width 3.5) (layer "B.Cu") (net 3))
 (segment (start 77.919998 65.159999) (end 67.139999 65.159999) (width 3.5) (layer "B.Cu") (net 3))
 (segment (start 57.13 63.369999) (end 58.92 65.159999) (width 5) (layer "F.Cu") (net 21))
 (segment (start 57.13 60.15) (end 57.13 63.369999) (width 5) (layer "F.Cu") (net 21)))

